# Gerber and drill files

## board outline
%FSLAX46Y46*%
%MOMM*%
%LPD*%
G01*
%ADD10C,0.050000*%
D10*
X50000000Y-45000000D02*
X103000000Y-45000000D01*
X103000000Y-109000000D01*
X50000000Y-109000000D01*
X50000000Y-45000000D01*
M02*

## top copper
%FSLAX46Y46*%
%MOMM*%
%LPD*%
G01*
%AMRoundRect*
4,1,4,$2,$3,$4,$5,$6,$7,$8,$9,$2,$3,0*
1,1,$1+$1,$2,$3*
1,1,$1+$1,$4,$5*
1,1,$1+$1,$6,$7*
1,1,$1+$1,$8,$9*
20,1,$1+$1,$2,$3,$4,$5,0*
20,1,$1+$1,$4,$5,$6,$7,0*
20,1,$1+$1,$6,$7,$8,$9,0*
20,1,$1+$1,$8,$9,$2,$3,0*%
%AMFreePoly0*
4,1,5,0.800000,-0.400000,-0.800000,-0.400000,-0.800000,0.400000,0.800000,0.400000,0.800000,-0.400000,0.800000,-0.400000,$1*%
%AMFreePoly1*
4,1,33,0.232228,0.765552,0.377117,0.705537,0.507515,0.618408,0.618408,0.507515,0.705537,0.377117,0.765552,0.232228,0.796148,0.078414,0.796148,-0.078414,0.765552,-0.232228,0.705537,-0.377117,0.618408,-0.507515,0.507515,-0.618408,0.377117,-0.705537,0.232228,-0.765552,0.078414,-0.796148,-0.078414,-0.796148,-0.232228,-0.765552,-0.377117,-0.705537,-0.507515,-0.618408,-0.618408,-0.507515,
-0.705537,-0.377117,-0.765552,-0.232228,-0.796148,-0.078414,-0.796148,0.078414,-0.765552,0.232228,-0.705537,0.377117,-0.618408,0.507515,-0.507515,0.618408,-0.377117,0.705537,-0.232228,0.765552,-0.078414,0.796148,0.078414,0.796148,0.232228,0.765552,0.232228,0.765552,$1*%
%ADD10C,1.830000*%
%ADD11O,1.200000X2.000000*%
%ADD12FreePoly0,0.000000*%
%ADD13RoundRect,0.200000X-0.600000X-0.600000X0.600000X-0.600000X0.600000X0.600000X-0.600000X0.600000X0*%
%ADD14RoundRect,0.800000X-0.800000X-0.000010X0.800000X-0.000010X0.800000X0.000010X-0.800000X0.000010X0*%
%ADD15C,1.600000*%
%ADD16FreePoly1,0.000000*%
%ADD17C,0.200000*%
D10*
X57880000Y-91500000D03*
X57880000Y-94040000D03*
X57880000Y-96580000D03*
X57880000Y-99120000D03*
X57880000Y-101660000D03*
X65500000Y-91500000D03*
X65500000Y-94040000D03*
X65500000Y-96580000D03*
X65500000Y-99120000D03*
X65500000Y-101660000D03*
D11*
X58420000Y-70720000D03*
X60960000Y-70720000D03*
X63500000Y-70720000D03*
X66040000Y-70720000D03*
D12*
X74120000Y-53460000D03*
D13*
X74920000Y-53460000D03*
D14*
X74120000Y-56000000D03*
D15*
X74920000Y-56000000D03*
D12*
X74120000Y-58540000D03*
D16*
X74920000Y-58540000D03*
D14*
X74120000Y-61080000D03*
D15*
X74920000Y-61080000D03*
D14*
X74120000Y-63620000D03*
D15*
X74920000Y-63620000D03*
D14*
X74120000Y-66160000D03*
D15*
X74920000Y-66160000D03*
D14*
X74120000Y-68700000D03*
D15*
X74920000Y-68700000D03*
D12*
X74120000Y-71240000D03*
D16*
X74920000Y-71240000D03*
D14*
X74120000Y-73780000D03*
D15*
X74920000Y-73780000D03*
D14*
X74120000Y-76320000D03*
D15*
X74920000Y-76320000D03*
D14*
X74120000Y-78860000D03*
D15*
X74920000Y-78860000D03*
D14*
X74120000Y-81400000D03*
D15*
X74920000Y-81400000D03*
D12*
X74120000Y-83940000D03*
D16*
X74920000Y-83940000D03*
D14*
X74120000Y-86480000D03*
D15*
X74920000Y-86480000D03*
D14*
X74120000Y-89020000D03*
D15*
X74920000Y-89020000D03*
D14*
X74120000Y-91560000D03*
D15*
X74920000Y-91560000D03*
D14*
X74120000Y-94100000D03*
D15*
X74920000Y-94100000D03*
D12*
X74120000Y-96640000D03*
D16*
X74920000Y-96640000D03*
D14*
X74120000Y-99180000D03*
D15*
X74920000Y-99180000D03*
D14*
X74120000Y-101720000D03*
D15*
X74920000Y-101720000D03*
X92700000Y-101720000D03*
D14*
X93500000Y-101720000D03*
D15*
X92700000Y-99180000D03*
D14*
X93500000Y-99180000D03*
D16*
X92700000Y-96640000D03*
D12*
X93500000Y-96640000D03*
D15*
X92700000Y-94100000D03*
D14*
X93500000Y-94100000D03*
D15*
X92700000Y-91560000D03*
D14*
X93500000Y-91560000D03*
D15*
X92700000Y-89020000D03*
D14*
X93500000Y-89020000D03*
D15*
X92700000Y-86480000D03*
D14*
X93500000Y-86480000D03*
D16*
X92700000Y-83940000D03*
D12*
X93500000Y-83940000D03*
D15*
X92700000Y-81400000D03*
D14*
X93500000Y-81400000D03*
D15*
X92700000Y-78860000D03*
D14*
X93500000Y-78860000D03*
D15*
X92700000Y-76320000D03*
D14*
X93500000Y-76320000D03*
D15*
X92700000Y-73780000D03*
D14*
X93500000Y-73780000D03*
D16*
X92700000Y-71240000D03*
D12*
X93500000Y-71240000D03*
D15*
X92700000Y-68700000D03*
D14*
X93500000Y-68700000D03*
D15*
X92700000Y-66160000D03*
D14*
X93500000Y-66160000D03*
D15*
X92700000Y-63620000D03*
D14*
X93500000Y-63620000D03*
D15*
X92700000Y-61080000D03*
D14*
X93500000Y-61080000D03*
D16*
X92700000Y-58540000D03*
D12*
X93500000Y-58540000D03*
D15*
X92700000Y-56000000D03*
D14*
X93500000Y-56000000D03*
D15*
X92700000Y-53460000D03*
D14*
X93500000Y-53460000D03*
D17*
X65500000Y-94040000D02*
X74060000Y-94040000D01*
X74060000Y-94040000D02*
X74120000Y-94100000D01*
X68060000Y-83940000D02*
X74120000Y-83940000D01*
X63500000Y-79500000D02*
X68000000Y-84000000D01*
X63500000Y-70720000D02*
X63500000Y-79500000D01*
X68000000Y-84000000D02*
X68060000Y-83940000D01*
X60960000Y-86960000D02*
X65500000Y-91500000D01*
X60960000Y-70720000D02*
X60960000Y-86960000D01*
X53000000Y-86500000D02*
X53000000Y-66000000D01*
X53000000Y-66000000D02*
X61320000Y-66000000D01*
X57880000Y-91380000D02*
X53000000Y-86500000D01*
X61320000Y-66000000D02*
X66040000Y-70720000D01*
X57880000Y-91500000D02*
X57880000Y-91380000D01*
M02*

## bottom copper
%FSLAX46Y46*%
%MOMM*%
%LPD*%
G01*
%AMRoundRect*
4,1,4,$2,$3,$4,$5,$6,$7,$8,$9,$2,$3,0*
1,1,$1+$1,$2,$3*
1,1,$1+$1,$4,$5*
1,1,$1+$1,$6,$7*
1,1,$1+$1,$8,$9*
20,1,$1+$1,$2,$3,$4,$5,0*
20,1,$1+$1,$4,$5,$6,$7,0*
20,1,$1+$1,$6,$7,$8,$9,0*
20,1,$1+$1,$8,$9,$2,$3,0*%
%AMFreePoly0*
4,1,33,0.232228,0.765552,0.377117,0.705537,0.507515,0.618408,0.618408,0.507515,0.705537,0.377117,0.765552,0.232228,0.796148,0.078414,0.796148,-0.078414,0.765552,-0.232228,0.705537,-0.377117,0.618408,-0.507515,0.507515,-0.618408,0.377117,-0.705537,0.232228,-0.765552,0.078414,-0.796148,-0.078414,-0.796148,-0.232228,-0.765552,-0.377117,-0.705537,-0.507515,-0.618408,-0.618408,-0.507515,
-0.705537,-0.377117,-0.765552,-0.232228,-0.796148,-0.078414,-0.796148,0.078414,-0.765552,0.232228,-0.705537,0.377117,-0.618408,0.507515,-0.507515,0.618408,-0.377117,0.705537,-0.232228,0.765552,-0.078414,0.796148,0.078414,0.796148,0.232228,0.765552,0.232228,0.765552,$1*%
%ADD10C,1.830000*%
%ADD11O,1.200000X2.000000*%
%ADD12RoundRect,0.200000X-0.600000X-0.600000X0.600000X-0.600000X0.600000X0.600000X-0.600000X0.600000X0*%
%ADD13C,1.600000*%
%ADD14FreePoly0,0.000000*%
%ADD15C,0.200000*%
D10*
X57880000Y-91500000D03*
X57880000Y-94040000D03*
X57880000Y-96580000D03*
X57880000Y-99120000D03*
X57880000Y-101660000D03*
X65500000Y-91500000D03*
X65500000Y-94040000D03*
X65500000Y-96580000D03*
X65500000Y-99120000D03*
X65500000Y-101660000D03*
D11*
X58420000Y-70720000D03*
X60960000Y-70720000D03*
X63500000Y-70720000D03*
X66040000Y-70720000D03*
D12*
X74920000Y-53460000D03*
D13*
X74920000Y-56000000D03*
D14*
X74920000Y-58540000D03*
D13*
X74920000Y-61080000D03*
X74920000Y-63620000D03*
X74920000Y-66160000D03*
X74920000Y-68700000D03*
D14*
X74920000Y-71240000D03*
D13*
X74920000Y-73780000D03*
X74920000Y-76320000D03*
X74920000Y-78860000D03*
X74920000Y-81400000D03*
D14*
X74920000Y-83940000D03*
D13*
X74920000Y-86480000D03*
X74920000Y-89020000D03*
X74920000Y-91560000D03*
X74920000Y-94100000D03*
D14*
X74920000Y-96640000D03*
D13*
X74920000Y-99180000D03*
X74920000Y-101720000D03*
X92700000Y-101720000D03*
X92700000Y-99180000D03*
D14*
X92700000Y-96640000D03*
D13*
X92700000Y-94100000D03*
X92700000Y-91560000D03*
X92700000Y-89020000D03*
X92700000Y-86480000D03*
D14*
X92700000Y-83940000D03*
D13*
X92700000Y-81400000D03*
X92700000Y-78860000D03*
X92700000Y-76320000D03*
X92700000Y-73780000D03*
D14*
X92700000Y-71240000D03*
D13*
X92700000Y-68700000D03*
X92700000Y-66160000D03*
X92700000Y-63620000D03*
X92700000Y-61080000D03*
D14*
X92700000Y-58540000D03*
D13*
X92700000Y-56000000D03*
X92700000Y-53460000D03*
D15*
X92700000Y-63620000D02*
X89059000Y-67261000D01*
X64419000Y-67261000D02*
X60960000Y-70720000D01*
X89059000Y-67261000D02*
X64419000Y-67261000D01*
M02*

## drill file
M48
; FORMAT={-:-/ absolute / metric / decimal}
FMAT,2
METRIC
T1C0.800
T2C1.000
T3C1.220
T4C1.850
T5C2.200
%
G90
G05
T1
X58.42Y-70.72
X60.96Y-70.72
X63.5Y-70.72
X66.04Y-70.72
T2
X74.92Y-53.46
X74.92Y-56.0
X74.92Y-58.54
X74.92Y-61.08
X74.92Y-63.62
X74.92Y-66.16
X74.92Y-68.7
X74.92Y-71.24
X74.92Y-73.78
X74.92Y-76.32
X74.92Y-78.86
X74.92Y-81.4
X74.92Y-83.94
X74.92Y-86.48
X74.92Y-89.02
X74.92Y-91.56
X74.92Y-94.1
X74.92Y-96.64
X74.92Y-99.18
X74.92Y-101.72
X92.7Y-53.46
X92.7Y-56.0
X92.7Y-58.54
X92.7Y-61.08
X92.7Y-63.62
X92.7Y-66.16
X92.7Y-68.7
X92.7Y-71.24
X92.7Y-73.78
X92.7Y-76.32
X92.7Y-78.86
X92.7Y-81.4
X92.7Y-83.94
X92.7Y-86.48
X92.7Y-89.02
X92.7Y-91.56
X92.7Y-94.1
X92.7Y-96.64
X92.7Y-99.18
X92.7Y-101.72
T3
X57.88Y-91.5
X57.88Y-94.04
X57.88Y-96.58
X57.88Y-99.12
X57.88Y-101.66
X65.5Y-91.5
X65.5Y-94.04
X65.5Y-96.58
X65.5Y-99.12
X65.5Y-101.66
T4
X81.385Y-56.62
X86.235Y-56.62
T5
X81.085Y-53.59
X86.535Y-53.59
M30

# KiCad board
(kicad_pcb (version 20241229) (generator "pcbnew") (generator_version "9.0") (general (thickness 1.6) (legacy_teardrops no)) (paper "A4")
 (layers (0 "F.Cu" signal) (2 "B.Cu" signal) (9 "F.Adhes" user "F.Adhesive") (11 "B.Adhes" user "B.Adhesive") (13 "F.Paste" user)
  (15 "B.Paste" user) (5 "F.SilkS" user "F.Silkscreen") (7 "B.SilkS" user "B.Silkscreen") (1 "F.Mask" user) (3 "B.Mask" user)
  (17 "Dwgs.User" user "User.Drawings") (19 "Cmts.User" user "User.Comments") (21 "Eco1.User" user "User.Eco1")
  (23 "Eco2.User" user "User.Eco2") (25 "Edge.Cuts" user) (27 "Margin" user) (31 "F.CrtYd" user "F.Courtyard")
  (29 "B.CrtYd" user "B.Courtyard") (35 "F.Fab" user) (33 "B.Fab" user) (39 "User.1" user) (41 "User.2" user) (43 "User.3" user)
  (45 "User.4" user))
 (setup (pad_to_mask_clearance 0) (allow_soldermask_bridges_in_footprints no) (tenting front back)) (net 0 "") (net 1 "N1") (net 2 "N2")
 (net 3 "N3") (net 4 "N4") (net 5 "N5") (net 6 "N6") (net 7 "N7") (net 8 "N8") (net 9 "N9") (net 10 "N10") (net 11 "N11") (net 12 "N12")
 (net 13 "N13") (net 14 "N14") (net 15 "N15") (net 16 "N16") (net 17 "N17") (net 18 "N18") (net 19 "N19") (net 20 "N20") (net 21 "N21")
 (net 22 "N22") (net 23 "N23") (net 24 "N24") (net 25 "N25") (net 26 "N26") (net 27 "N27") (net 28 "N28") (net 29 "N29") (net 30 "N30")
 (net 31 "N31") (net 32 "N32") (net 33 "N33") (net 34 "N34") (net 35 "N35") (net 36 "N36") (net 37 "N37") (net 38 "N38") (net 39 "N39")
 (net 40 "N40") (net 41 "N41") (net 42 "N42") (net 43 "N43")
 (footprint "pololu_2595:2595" (layer "F.Cu") (at 57.88 91.5)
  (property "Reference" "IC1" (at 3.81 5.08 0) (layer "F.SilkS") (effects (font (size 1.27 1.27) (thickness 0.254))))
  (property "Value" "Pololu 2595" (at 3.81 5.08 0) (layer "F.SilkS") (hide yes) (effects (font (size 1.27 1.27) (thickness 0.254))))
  (pad "1" thru_hole circle (at 0 0) (size 1.83 1.83) (drill 1.22) (layers "*.Cu" "*.Mask") (remove_unused_layers no) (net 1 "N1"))
  (pad "2" thru_hole circle (at 0 2.54) (size 1.83 1.83) (drill 1.22) (layers "*.Cu" "*.Mask") (remove_unused_layers no) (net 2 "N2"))
  (pad "3" thru_hole circle (at 0 5.08) (size 1.83 1.83) (drill 1.22) (layers "*.Cu" "*.Mask") (remove_unused_layers no) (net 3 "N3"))
  (pad "4" thru_hole circle (at 0 7.62) (size 1.83 1.83) (drill 1.22) (layers "*.Cu" "*.Mask") (remove_unused_layers no) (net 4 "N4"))
  (pad "5" thru_hole circle (at 0 10.16) (size 1.83 1.83) (drill 1.22) (layers "*.Cu" "*.Mask") (remove_unused_layers no) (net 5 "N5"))
  (pad "6" thru_hole circle (at 7.62 0) (size 1.83 1.83) (drill 1.22) (layers "*.Cu" "*.Mask") (remove_unused_layers no) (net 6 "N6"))
  (pad "7" thru_hole circle (at 7.62 2.54) (size 1.83 1.83) (drill 1.22) (layers "*.Cu" "*.Mask") (remove_unused_layers no) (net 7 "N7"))
  (pad "8" thru_hole circle (at 7.62 5.08) (size 1.83 1.83) (drill 1.22) (layers "*.Cu" "*.Mask") (remove_unused_layers no) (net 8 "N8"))
  (pad "9" thru_hole circle (at 7.62 7.62) (size 1.83 1.83) (drill 1.22) (layers "*.Cu" "*.Mask") (remove_unused_layers no) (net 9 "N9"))
  (pad "10" thru_hole circle (at 7.62 10.16) (size 1.83 1.83) (drill 1.22) (layers "*.Cu" "*.Mask") (remove_unused_layers no) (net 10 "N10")))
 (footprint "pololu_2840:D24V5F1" (layer "F.Cu") (at 62.23 70.72)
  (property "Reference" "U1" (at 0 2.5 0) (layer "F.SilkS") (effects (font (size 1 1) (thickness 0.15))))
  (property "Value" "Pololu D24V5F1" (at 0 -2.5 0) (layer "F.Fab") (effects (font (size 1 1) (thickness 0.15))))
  (pad "1" thru_hole oval (at -3.81 0) (size 1.2 2) (drill 0.8) (layers "*.Cu" "*.Mask") (remove_unused_layers no) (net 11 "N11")
   (thermal_bridge_angle 45))
  (pad "2" thru_hole oval (at -1.27 0) (size 1.2 2) (drill 0.8) (layers "*.Cu" "*.Mask") (remove_unused_layers no) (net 6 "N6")
   (thermal_bridge_angle 45))
  (pad "3" thru_hole oval (at 1.27 0) (size 1.2 2) (drill 0.8) (layers "*.Cu" "*.Mask") (remove_unused_layers no) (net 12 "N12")
   (thermal_bridge_angle 45))
  (pad "4" thru_hole oval (at 3.81 0) (size 1.2 2) (drill 0.8) (layers "*.Cu" "*.Mask") (remove_unused_layers no) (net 1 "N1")
   (thermal_bridge_angle 45)))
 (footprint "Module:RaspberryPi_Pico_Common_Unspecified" (layer "F.Cu") (at 83.81 77.59)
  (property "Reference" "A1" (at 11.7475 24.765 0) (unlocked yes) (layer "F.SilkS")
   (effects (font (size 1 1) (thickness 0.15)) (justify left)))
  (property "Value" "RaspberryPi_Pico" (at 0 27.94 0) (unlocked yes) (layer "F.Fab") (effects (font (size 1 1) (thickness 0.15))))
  (pad "" np_thru_hole circle (at -2.725 -24) (size 2.2 2.2) (drill 2.2) (layers "*.Mask"))
  (pad "" np_thru_hole circle (at -2.425 -20.97) (size 1.85 1.85) (drill 1.85) (layers "*.Mask"))
  (pad "" np_thru_hole circle (at 2.425 -20.97) (size 1.85 1.85) (drill 1.85) (layers "*.Mask"))
  (pad "" np_thru_hole circle (at 2.725 -24) (size 2.2 2.2) (drill 2.2) (layers "*.Mask"))
  (pad "1" smd custom (at -9.69 -24.13) (size 1.6 0.8) (layers "F.Cu" "F.Mask") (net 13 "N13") (options (clearance outline) (anchor rect))
   (primitives))
  (pad "1" thru_hole roundrect (at -8.89 -24.13) (size 1.6 1.6) (drill 1) (layers "*.Cu" "*.Mask") (remove_unused_layers no)
   (roundrect_rratio 0.125) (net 13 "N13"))
  (pad "2" smd roundrect (at -9.69 -21.59) (size 3.2 1.6) (layers "F.Cu" "F.Mask") (roundrect_rratio 0.5) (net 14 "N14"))
  (pad "2" thru_hole circle (at -8.89 -21.59) (size 1.6 1.6) (drill 1) (layers "*.Cu" "*.Mask") (remove_unused_layers no) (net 14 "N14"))
  (pad "3" smd custom (at -9.69 -19.05) (size 1.6 0.8) (layers "F.Cu" "F.Mask") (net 12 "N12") (options (clearance outline) (anchor rect))
   (primitives))
  (pad "3" thru_hole custom (at -8.89 -19.05) (size 1.6 1.6) (drill 1) (layers "*.Cu" "*.Mask") (remove_unused_layers no) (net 12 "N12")
   (options (clearance outline) (anchor circle)) (primitives))
  (pad "4" smd roundrect (at -9.69 -16.51) (size 3.2 1.6) (layers "F.Cu" "F.Mask") (roundrect_rratio 0.5) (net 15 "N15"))
  (pad "4" thru_hole circle (at -8.89 -16.51) (size 1.6 1.6) (drill 1) (layers "*.Cu" "*.Mask") (remove_unused_layers no) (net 15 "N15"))
  (pad "5" smd roundrect (at -9.69 -13.97) (size 3.2 1.6) (layers "F.Cu" "F.Mask") (roundrect_rratio 0.5) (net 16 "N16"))
  (pad "5" thru_hole circle (at -8.89 -13.97) (size 1.6 1.6) (drill 1) (layers "*.Cu" "*.Mask") (remove_unused_layers no) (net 16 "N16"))
  (pad "6" smd roundrect (at -9.69 -11.43) (size 3.2 1.6) (layers "F.Cu" "F.Mask") (roundrect_rratio 0.5) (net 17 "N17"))
  (pad "6" thru_hole circle (at -8.89 -11.43) (size 1.6 1.6) (drill 1) (layers "*.Cu" "*.Mask") (remove_unused_layers no) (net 17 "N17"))
  (pad "7" smd roundrect (at -9.69 -8.89) (size 3.2 1.6) (layers "F.Cu" "F.Mask") (roundrect_rratio 0.5) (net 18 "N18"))
  (pad "7" thru_hole circle (at -8.89 -8.89) (size 1.6 1.6) (drill 1) (layers "*.Cu" "*.Mask") (remove_unused_layers no) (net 18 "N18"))
  (pad "8" smd custom (at -9.69 -6.35) (size 1.6 0.8) (layers "F.Cu" "F.Mask") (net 12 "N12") (options (clearance outline) (anchor rect))
   (primitives))
  (pad "8" thru_hole custom (at -8.89 -6.35) (size 1.6 1.6) (drill 1) (layers "*.Cu" "*.Mask") (remove_unused_layers no) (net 12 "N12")
   (options (clearance outline) (anchor circle)) (primitives))
  (pad "9" smd roundrect (at -9.69 -3.81) (size 3.2 1.6) (layers "F.Cu" "F.Mask") (roundrect_rratio 0.5) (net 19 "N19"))
  (pad "9" thru_hole circle (at -8.89 -3.81) (size 1.6 1.6) (drill 1) (layers "*.Cu" "*.Mask") (remove_unused_layers no) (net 19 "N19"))
  (pad "10" smd roundrect (at -9.69 -1.27) (size 3.2 1.6) (layers "F.Cu" "F.Mask") (roundrect_rratio 0.5) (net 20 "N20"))
  (pad "10" thru_hole circle (at -8.89 -1.27) (size 1.6 1.6) (drill 1) (layers "*.Cu" "*.Mask") (remove_unused_layers no) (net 20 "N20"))
  (pad "11" smd roundrect (at -9.69 1.27) (size 3.2 1.6) (layers "F.Cu" "F.Mask") (roundrect_rratio 0.5) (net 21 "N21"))
  (pad "11" thru_hole circle (at -8.89 1.27) (size 1.6 1.6) (drill 1) (layers "*.Cu" "*.Mask") (remove_unused_layers no) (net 21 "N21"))
  (pad "12" smd roundrect (at -9.69 3.81) (size 3.2 1.6) (layers "F.Cu" "F.Mask") (roundrect_rratio 0.5) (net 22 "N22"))
  (pad "12" thru_hole circle (at -8.89 3.81) (size 1.6 1.6) (drill 1) (layers "*.Cu" "*.Mask") (remove_unused_layers no) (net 22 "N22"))
  (pad "13" smd custom (at -9.69 6.35) (size 1.6 0.8) (layers "F.Cu" "F.Mask") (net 12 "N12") (options (clearance outline) (anchor rect))
   (primitives))
  (pad "13" thru_hole custom (at -8.89 6.35) (size 1.6 1.6) (drill 1) (layers "*.Cu" "*.Mask") (remove_unused_layers no) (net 12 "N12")
   (options (clearance outline) (anchor circle)) (primitives))
  (pad "14" smd roundrect (at -9.69 8.89) (size 3.2 1.6) (layers "F.Cu" "F.Mask") (roundrect_rratio 0.5) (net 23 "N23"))
  (pad "14" thru_hole circle (at -8.89 8.89) (size 1.6 1.6) (drill 1) (layers "*.Cu" "*.Mask") (remove_unused_layers no) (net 23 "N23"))
  (pad "15" smd roundrect (at -9.69 11.43) (size 3.2 1.6) (layers "F.Cu" "F.Mask") (roundrect_rratio 0.5) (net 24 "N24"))
  (pad "15" thru_hole circle (at -8.89 11.43) (size 1.6 1.6) (drill 1) (layers "*.Cu" "*.Mask") (remove_unused_layers no) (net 24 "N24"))
  (pad "16" smd roundrect (at -9.69 13.97) (size 3.2 1.6) (layers "F.Cu" "F.Mask") (roundrect_rratio 0.5) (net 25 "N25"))
  (pad "16" thru_hole circle (at -8.89 13.97) (size 1.6 1.6) (drill 1) (layers "*.Cu" "*.Mask") (remove_unused_layers no) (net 25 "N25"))
  (pad "17" smd roundrect (at -9.69 16.51) (size 3.2 1.6) (layers "F.Cu" "F.Mask") (roundrect_rratio 0.5) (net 7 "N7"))
  (pad "17" thru_hole circle (at -8.89 16.51) (size 1.6 1.6) (drill 1) (layers "*.Cu" "*.Mask") (remove_unused_layers no) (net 7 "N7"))
  (pad "18" smd custom (at -9.69 19.05) (size 1.6 0.8) (layers "F.Cu" "F.Mask") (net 12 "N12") (options (clearance outline) (anchor rect))
   (primitives))
  (pad "18" thru_hole custom (at -8.89 19.05) (size 1.6 1.6) (drill 1) (layers "*.Cu" "*.Mask") (remove_unused_layers no) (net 12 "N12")
   (options (clearance outline) (anchor circle)) (primitives))
  (pad "19" smd roundrect (at -9.69 21.59) (size 3.2 1.6) (layers "F.Cu" "F.Mask") (roundrect_rratio 0.5) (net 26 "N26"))
  (pad "19" thru_hole circle (at -8.89 21.59) (size 1.6 1.6) (drill 1) (layers "*.Cu" "*.Mask") (remove_unused_layers no) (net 26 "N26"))
  (pad "20" smd roundrect (at -9.69 24.13) (size 3.2 1.6) (layers "F.Cu" "F.Mask") (roundrect_rratio 0.5) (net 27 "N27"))
  (pad "20" thru_hole circle (at -8.89 24.13) (size 1.6 1.6) (drill 1) (layers "*.Cu" "*.Mask") (remove_unused_layers no) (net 27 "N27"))
  (pad "21" thru_hole circle (at 8.89 24.13) (size 1.6 1.6) (drill 1) (layers "*.Cu" "*.Mask") (remove_unused_layers no) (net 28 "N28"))
  (pad "21" smd roundrect (at 9.69 24.13) (size 3.2 1.6) (layers "F.Cu" "F.Mask") (roundrect_rratio 0.5) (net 28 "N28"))
  (pad "22" thru_hole circle (at 8.89 21.59) (size 1.6 1.6) (drill 1) (layers "*.Cu" "*.Mask") (remove_unused_layers no) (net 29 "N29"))
  (pad "22" smd roundrect (at 9.69 21.59) (size 3.2 1.6) (layers "F.Cu" "F.Mask") (roundrect_rratio 0.5) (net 29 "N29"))
  (pad "23" thru_hole custom (at 8.89 19.05) (size 1.6 1.6) (drill 1) (layers "*.Cu" "*.Mask") (remove_unused_layers no) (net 12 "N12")
   (options (clearance outline) (anchor circle)) (primitives))
  (pad "23" smd custom (at 9.69 19.05) (size 1.6 0.8) (layers "F.Cu" "F.Mask") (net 12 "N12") (options (clearance outline) (anchor rect))
   (primitives))
  (pad "24" thru_hole circle (at 8.89 16.51) (size 1.6 1.6) (drill 1) (layers "*.Cu" "*.Mask") (remove_unused_layers no) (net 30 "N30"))
  (pad "24" smd roundrect (at 9.69 16.51) (size 3.2 1.6) (layers "F.Cu" "F.Mask") (roundrect_rratio 0.5) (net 30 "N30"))
  (pad "25" thru_hole circle (at 8.89 13.97) (size 1.6 1.6) (drill 1) (layers "*.Cu" "*.Mask") (remove_unused_layers no) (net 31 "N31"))
  (pad "25" smd roundrect (at 9.69 13.97) (size 3.2 1.6) (layers "F.Cu" "F.Mask") (roundrect_rratio 0.5) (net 31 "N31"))
  (pad "26" thru_hole circle (at 8.89 11.43) (size 1.6 1.6) (drill 1) (layers "*.Cu" "*.Mask") (remove_unused_layers no) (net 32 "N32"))
  (pad "26" smd roundrect (at 9.69 11.43) (size 3.2 1.6) (layers "F.Cu" "F.Mask") (roundrect_rratio 0.5) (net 32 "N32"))
  (pad "27" thru_hole circle (at 8.89 8.89) (size 1.6 1.6) (drill 1) (layers "*.Cu" "*.Mask") (remove_unused_layers no) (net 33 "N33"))
  (pad "27" smd roundrect (at 9.69 8.89) (size 3.2 1.6) (layers "F.Cu" "F.Mask") (roundrect_rratio 0.5) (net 33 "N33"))
  (pad "28" thru_hole custom (at 8.89 6.35) (size 1.6 1.6) (drill 1) (layers "*.Cu" "*.Mask") (remove_unused_layers no) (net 12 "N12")
   (options (clearance outline) (anchor circle)) (primitives))
  (pad "28" smd custom (at 9.69 6.35) (size 1.6 0.8) (layers "F.Cu" "F.Mask") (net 12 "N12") (options (clearance outline) (anchor rect))
   (primitives))
  (pad "29" thru_hole circle (at 8.89 3.81) (size 1.6 1.6) (drill 1) (layers "*.Cu" "*.Mask") (remove_unused_layers no) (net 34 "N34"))
  (pad "29" smd roundrect (at 9.69 3.81) (size 3.2 1.6) (layers "F.Cu" "F.Mask") (roundrect_rratio 0.5) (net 34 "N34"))
  (pad "30" thru_hole circle (at 8.89 1.27) (size 1.6 1.6) (drill 1) (layers "*.Cu" "*.Mask") (remove_unused_layers no) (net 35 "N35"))
  (pad "30" smd roundrect (at 9.69 1.27) (size 3.2 1.6) (layers "F.Cu" "F.Mask") (roundrect_rratio 0.5) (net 35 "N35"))
  (pad "31" thru_hole circle (at 8.89 -1.27) (size 1.6 1.6) (drill 1) (layers "*.Cu" "*.Mask") (remove_unused_layers no) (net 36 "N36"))
  (pad "31" smd roundrect (at 9.69 -1.27) (size 3.2 1.6) (layers "F.Cu" "F.Mask") (roundrect_rratio 0.5) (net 36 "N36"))
  (pad "32" thru_hole circle (at 8.89 -3.81) (size 1.6 1.6) (drill 1) (layers "*.Cu" "*.Mask") (remove_unused_layers no) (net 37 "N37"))
  (pad "32" smd roundrect (at 9.69 -3.81) (size 3.2 1.6) (layers "F.Cu" "F.Mask") (roundrect_rratio 0.5) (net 37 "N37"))
  (pad "33" thru_hole custom (at 8.89 -6.35) (size 1.6 1.6) (drill 1) (layers "*.Cu" "*.Mask") (remove_unused_layers no) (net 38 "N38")
   (options (clearance outline) (anchor circle)) (primitives))
  (pad "33" smd custom (at 9.69 -6.35) (size 1.6 0.8) (layers "F.Cu" "F.Mask") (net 38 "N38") (options (clearance outline) (anchor rect))
   (primitives))
  (pad "34" thru_hole circle (at 8.89 -8.89) (size 1.6 1.6) (drill 1) (layers "*.Cu" "*.Mask") (remove_unused_layers no) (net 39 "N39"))
  (pad "34" smd roundrect (at 9.69 -8.89) (size 3.2 1.6) (layers "F.Cu" "F.Mask") (roundrect_rratio 0.5) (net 39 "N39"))
  (pad "35" thru_hole circle (at 8.89 -11.43) (size 1.6 1.6) (drill 1) (layers "*.Cu" "*.Mask") (remove_unused_layers no) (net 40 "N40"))
  (pad "35" smd roundrect (at 9.69 -11.43) (size 3.2 1.6) (layers "F.Cu" "F.Mask") (roundrect_rratio 0.5) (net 40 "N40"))
  (pad "36" thru_hole circle (at 8.89 -13.97) (size 1.6 1.6) (drill 1) (layers "*.Cu" "*.Mask") (remove_unused_layers no) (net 6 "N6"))
  (pad "36" smd roundrect (at 9.69 -13.97) (size 3.2 1.6) (layers "F.Cu" "F.Mask") (roundrect_rratio 0.5) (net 6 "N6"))
  (pad "37" thru_hole circle (at 8.89 -16.51) (size 1.6 1.6) (drill 1) (layers "*.Cu" "*.Mask") (remove_unused_layers no) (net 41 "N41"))
  (pad "37" smd roundrect (at 9.69 -16.51) (size 3.2 1.6) (layers "F.Cu" "F.Mask") (roundrect_rratio 0.5) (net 41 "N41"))
  (pad "38" thru_hole custom (at 8.89 -19.05) (size 1.6 1.6) (drill 1) (layers "*.Cu" "*.Mask") (remove_unused_layers no) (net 12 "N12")
   (options (clearance outline) (anchor circle)) (primitives))
  (pad "38" smd custom (at 9.69 -19.05) (size 1.6 0.8) (layers "F.Cu" "F.Mask") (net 12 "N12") (options (clearance outline) (anchor rect))
   (primitives))
  (pad "39" thru_hole circle (at 8.89 -21.59) (size 1.6 1.6) (drill 1) (layers "*.Cu" "*.Mask") (remove_unused_layers no) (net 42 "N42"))
  (pad "39" smd roundrect (at 9.69 -21.59) (size 3.2 1.6) (layers "F.Cu" "F.Mask") (roundrect_rratio 0.5) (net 42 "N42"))
  (pad "40" thru_hole circle (at 8.89 -24.13) (size 1.6 1.6) (drill 1) (layers "*.Cu" "*.Mask") (remove_unused_layers no) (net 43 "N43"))
  (pad "40" smd roundrect (at 9.69 -24.13) (size 3.2 1.6) (layers "F.Cu" "F.Mask") (roundrect_rratio 0.5) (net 43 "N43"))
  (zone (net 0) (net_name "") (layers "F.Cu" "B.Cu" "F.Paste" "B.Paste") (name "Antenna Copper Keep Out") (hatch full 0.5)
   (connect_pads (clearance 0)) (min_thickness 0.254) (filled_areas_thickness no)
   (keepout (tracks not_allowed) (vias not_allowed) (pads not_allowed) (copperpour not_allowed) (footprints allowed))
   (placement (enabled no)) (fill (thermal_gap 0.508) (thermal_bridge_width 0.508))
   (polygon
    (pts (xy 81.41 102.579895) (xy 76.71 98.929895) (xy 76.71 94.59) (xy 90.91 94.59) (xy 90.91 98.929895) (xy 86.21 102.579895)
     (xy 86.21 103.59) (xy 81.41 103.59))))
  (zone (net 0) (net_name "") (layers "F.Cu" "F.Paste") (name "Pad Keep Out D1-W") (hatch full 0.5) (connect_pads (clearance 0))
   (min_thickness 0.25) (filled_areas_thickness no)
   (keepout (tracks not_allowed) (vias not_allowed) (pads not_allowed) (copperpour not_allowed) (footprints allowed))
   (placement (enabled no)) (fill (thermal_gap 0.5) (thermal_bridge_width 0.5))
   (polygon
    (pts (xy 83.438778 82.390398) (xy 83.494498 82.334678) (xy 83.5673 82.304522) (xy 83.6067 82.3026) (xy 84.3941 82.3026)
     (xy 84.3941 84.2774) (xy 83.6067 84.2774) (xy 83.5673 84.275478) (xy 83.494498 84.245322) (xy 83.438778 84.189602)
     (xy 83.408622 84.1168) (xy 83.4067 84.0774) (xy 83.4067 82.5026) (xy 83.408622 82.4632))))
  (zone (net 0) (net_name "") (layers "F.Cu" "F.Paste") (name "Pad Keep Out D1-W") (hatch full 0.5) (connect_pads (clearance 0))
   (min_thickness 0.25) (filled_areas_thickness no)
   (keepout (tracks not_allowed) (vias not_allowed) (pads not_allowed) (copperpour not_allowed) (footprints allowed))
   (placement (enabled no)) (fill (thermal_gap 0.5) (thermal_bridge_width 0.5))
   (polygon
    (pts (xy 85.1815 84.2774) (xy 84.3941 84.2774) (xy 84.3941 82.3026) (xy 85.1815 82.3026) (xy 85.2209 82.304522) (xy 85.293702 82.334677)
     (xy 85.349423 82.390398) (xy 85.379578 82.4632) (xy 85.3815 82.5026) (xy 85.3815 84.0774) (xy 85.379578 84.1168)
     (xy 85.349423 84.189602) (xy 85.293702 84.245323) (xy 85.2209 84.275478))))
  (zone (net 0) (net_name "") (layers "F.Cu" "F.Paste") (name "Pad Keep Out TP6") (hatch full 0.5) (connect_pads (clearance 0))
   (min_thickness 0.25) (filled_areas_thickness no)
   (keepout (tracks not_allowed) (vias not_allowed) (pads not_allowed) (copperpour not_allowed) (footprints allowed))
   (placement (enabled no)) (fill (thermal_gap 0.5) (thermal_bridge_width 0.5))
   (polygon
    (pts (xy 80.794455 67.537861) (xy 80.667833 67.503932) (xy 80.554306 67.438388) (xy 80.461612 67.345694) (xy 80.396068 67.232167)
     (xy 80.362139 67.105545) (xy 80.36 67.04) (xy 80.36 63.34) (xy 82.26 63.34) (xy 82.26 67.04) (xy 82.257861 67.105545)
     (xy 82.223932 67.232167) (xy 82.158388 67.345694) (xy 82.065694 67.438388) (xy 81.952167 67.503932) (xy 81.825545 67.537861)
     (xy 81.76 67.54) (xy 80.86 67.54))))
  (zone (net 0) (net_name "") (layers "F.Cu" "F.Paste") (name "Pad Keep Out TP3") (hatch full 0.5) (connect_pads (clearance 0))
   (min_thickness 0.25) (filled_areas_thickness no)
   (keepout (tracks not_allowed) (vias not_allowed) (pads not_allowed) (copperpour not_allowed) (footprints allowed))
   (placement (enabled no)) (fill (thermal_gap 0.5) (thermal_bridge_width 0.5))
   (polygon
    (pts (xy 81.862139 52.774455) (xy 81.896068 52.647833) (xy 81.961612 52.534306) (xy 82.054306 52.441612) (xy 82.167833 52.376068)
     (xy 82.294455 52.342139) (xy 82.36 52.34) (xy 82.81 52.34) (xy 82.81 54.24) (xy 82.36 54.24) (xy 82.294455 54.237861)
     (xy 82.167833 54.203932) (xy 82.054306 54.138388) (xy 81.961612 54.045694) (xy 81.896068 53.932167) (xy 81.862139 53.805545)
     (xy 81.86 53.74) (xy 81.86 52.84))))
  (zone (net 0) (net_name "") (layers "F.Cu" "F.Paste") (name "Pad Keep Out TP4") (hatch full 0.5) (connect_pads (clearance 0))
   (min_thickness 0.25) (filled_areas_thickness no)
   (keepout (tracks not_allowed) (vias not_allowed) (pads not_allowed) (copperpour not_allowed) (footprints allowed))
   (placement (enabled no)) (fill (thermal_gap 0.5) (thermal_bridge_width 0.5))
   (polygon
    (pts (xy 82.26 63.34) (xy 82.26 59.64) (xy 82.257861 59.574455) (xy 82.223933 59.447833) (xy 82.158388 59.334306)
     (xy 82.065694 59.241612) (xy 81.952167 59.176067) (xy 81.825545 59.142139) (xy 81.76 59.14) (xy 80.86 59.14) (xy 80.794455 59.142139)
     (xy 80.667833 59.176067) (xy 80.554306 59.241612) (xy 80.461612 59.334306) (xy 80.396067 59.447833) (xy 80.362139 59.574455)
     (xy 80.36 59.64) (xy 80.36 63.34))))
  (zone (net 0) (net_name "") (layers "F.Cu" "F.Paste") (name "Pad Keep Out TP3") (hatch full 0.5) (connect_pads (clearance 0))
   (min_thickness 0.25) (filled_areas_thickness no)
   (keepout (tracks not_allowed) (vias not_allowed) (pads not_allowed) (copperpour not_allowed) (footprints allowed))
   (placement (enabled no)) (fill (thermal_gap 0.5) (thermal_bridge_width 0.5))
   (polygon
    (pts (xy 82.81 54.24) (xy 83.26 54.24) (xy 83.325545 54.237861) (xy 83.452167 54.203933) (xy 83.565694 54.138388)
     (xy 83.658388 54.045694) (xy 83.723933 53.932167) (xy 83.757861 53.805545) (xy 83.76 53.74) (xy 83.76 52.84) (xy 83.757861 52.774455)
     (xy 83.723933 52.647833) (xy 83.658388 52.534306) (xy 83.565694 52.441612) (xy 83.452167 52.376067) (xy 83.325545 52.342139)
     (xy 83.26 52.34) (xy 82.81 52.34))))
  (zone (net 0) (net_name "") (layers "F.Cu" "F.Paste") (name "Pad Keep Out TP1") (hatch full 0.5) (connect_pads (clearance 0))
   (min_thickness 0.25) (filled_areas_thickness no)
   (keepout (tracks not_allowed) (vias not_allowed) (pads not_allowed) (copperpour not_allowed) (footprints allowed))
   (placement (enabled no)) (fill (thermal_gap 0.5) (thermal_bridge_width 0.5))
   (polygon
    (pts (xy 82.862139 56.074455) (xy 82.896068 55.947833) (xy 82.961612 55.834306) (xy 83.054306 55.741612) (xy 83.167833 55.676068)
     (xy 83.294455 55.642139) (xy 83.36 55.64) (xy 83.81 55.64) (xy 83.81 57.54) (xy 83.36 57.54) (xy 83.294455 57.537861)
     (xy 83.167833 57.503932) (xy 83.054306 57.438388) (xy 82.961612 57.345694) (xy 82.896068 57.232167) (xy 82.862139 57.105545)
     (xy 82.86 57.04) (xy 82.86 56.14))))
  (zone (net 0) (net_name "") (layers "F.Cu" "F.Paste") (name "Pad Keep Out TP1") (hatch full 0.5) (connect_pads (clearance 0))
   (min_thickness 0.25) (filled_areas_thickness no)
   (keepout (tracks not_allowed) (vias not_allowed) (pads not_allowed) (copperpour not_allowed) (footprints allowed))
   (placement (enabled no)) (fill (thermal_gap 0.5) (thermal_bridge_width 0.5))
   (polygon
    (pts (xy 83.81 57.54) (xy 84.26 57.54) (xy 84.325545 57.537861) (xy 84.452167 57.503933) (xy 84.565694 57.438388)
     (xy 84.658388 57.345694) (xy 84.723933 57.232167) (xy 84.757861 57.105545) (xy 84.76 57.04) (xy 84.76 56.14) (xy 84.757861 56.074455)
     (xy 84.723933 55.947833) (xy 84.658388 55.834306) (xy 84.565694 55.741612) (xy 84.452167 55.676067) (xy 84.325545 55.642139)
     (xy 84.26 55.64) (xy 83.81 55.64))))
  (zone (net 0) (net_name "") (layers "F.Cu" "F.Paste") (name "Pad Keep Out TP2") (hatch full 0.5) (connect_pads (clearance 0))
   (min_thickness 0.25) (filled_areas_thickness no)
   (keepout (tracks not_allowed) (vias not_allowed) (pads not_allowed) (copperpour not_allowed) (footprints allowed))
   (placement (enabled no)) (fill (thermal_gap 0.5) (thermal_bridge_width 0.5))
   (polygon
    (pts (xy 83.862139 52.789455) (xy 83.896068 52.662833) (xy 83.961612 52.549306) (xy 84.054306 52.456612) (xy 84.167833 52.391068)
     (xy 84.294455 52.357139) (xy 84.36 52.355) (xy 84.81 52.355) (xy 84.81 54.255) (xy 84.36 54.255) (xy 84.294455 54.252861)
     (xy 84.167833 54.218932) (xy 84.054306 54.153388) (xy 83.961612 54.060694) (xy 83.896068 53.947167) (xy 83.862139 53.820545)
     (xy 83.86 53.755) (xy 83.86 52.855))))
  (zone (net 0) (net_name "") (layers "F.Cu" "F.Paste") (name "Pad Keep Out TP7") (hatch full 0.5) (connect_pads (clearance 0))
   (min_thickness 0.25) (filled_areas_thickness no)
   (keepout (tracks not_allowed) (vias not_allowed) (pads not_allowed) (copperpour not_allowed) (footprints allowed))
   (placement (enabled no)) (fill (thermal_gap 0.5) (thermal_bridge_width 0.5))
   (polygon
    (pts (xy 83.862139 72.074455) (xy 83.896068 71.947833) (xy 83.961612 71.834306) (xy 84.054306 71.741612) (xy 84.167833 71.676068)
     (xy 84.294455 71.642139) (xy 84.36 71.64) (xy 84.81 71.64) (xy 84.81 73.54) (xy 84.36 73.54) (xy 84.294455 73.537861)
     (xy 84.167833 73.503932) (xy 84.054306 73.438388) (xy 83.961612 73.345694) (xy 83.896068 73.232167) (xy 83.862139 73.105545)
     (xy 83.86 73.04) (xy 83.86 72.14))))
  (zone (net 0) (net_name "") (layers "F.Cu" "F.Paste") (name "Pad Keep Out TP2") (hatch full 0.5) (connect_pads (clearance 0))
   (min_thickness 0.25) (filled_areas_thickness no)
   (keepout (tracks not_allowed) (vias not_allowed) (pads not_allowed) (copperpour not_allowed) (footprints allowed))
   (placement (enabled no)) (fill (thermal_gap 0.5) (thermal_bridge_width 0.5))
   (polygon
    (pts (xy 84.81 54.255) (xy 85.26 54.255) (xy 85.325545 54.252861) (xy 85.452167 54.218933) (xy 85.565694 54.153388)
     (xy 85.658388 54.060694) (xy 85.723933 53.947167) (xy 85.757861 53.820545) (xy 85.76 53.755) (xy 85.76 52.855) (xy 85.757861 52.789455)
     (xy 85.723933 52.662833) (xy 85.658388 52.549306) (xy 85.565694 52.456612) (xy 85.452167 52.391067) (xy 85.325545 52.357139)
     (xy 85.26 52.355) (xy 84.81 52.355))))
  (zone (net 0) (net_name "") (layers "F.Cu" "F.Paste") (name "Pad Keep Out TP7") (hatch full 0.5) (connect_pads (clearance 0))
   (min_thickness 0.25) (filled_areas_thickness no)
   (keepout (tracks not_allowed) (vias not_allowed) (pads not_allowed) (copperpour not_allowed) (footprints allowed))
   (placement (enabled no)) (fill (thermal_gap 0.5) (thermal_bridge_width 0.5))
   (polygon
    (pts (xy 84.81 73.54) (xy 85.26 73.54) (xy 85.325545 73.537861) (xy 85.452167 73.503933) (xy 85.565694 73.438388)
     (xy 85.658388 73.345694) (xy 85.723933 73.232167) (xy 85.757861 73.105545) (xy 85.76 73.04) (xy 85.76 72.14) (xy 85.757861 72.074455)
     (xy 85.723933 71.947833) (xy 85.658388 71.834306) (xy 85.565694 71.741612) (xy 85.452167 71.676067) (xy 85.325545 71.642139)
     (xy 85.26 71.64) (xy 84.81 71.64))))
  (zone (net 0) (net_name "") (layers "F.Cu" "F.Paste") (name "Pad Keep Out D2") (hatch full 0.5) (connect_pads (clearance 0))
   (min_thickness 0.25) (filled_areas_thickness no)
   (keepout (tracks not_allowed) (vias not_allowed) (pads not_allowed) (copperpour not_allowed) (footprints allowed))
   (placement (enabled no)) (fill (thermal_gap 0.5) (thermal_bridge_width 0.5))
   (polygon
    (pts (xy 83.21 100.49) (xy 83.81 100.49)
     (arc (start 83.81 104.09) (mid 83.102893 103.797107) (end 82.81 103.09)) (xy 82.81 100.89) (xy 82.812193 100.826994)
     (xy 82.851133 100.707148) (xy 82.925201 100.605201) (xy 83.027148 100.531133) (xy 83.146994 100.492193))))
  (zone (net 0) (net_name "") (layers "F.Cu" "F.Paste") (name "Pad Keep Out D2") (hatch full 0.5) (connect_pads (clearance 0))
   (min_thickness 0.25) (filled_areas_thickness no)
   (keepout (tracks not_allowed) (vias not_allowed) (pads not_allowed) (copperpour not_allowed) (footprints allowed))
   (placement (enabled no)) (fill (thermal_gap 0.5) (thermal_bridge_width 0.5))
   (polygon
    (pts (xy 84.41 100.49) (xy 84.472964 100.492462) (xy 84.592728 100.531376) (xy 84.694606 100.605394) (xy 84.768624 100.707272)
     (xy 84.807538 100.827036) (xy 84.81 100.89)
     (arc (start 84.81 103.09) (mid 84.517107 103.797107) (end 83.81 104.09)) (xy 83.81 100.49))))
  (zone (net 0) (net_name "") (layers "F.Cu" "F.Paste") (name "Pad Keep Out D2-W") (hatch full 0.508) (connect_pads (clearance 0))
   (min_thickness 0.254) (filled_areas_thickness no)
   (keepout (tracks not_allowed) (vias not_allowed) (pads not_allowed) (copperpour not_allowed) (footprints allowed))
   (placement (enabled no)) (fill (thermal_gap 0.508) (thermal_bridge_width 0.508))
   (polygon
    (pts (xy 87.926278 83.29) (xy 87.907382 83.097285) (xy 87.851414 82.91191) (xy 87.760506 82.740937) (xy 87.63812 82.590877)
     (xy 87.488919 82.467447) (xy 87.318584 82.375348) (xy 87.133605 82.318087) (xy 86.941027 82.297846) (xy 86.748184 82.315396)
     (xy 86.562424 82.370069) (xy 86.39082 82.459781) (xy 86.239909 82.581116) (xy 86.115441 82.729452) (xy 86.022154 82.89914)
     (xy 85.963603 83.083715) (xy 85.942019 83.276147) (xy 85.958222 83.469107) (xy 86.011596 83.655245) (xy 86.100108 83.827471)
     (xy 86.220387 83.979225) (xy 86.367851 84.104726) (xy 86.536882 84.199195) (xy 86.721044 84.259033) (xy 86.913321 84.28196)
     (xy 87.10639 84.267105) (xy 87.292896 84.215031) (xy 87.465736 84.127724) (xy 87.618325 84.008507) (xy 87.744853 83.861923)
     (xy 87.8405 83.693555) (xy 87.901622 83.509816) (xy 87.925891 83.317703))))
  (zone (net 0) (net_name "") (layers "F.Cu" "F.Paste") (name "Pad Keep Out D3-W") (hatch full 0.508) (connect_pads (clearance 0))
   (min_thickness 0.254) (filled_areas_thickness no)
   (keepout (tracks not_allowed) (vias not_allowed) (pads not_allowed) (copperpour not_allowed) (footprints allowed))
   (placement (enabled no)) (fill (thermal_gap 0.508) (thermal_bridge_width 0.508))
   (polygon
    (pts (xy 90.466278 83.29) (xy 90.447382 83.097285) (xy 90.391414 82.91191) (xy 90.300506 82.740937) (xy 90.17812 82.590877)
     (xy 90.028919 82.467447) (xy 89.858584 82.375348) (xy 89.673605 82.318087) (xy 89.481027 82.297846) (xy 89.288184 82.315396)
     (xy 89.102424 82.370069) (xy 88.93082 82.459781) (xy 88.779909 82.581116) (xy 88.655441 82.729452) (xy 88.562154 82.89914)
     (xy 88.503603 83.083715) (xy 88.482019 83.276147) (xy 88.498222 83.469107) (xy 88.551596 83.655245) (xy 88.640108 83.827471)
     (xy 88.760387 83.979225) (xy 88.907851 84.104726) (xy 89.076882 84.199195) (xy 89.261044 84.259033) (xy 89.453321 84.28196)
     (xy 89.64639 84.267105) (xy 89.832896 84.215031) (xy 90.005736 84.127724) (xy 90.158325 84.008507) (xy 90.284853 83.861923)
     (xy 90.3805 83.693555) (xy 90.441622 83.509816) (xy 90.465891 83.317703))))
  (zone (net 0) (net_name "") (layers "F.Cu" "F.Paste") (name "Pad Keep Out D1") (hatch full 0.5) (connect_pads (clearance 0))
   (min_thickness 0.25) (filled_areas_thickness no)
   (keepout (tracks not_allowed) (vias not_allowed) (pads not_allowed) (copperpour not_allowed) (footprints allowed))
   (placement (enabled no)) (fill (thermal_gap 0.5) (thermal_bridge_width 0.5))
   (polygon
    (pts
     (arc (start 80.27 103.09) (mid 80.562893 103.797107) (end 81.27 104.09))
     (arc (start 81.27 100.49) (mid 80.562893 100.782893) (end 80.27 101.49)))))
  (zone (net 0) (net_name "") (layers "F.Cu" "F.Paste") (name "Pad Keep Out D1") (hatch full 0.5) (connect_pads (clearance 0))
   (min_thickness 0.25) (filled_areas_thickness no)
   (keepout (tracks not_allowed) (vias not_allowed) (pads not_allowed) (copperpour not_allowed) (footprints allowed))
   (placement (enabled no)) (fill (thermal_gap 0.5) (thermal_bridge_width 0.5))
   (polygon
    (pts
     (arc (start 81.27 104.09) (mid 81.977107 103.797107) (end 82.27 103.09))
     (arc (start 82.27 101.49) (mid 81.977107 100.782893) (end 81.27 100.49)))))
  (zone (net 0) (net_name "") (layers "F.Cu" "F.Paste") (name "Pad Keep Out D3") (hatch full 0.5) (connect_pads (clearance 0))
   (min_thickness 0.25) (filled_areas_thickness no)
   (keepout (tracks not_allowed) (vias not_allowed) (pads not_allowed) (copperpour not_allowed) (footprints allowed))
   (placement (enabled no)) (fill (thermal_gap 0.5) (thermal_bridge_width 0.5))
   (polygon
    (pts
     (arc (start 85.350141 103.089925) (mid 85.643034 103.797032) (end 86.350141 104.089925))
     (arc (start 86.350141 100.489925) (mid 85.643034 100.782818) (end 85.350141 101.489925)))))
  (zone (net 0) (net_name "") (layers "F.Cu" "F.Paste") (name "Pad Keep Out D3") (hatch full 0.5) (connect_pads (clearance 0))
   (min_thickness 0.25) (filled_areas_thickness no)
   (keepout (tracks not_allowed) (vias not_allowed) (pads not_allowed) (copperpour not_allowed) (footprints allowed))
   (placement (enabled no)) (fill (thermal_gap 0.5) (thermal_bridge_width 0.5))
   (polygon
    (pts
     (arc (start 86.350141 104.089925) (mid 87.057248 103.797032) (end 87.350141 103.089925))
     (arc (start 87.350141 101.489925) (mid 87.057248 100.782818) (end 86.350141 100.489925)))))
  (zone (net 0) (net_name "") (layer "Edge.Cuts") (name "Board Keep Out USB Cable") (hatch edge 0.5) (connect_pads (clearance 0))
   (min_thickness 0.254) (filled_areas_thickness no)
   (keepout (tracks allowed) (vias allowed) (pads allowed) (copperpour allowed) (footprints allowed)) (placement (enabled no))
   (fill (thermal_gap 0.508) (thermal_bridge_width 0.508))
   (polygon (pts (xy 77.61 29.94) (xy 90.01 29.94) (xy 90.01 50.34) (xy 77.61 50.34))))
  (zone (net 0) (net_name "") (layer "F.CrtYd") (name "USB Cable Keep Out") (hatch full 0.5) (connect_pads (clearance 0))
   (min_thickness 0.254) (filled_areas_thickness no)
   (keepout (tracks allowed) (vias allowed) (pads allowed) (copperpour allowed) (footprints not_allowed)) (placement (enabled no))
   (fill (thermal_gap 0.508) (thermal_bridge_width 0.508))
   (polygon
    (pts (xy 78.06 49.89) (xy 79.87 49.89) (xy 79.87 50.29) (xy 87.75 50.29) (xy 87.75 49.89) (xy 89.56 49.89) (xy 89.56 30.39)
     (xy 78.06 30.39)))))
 (gr_rect (start 50 45) (end 103 109) (stroke (width 0.05) (type default)) (fill no) (layer "Edge.Cuts"))
 (segment (start 65.5 94.04) (end 74.06 94.04) (width 0.2) (layer "F.Cu") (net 7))
 (segment (start 74.06 94.04) (end 74.12 94.1) (width 0.2) (layer "F.Cu") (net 7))
 (segment (start 68.06 83.94) (end 74.12 83.94) (width 0.2) (layer "F.Cu") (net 12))
 (segment (start 63.5 79.5) (end 68 84) (width 0.2) (layer "F.Cu") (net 12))
 (segment (start 63.5 70.72) (end 63.5 79.5) (width 0.2) (layer "F.Cu") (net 12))
 (segment (start 68 84) (end 68.06 83.94) (width 0.2) (layer "F.Cu") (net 12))
 (segment (start 60.96 86.96) (end 65.5 91.5) (width 0.2) (layer "F.Cu") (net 6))
 (segment (start 60.96 70.72) (end 60.96 86.96) (width 0.2) (layer "F.Cu") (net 6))
 (segment (start 92.7 63.62) (end 89.059 67.261) (width 0.2) (layer "B.Cu") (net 6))
 (segment (start 64.419 67.261) (end 60.96 70.72) (width 0.2) (layer "B.Cu") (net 6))
 (segment (start 89.059 67.261) (end 64.419 67.261) (width 0.2) (layer "B.Cu") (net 6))
 (segment (start 53 86.5) (end 53 66) (width 0.2) (layer "F.Cu") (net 1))
 (segment (start 53 66) (end 61.32 66) (width 0.2) (layer "F.Cu") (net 1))
 (segment (start 57.88 91.38) (end 53 86.5) (width 0.2) (layer "F.Cu") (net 1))
 (segment (start 61.32 66) (end 66.04 70.72) (width 0.2) (layer "F.Cu") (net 1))
 (segment (start 57.88 91.5) (end 57.88 91.38) (width 0.2) (layer "F.Cu") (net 1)))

